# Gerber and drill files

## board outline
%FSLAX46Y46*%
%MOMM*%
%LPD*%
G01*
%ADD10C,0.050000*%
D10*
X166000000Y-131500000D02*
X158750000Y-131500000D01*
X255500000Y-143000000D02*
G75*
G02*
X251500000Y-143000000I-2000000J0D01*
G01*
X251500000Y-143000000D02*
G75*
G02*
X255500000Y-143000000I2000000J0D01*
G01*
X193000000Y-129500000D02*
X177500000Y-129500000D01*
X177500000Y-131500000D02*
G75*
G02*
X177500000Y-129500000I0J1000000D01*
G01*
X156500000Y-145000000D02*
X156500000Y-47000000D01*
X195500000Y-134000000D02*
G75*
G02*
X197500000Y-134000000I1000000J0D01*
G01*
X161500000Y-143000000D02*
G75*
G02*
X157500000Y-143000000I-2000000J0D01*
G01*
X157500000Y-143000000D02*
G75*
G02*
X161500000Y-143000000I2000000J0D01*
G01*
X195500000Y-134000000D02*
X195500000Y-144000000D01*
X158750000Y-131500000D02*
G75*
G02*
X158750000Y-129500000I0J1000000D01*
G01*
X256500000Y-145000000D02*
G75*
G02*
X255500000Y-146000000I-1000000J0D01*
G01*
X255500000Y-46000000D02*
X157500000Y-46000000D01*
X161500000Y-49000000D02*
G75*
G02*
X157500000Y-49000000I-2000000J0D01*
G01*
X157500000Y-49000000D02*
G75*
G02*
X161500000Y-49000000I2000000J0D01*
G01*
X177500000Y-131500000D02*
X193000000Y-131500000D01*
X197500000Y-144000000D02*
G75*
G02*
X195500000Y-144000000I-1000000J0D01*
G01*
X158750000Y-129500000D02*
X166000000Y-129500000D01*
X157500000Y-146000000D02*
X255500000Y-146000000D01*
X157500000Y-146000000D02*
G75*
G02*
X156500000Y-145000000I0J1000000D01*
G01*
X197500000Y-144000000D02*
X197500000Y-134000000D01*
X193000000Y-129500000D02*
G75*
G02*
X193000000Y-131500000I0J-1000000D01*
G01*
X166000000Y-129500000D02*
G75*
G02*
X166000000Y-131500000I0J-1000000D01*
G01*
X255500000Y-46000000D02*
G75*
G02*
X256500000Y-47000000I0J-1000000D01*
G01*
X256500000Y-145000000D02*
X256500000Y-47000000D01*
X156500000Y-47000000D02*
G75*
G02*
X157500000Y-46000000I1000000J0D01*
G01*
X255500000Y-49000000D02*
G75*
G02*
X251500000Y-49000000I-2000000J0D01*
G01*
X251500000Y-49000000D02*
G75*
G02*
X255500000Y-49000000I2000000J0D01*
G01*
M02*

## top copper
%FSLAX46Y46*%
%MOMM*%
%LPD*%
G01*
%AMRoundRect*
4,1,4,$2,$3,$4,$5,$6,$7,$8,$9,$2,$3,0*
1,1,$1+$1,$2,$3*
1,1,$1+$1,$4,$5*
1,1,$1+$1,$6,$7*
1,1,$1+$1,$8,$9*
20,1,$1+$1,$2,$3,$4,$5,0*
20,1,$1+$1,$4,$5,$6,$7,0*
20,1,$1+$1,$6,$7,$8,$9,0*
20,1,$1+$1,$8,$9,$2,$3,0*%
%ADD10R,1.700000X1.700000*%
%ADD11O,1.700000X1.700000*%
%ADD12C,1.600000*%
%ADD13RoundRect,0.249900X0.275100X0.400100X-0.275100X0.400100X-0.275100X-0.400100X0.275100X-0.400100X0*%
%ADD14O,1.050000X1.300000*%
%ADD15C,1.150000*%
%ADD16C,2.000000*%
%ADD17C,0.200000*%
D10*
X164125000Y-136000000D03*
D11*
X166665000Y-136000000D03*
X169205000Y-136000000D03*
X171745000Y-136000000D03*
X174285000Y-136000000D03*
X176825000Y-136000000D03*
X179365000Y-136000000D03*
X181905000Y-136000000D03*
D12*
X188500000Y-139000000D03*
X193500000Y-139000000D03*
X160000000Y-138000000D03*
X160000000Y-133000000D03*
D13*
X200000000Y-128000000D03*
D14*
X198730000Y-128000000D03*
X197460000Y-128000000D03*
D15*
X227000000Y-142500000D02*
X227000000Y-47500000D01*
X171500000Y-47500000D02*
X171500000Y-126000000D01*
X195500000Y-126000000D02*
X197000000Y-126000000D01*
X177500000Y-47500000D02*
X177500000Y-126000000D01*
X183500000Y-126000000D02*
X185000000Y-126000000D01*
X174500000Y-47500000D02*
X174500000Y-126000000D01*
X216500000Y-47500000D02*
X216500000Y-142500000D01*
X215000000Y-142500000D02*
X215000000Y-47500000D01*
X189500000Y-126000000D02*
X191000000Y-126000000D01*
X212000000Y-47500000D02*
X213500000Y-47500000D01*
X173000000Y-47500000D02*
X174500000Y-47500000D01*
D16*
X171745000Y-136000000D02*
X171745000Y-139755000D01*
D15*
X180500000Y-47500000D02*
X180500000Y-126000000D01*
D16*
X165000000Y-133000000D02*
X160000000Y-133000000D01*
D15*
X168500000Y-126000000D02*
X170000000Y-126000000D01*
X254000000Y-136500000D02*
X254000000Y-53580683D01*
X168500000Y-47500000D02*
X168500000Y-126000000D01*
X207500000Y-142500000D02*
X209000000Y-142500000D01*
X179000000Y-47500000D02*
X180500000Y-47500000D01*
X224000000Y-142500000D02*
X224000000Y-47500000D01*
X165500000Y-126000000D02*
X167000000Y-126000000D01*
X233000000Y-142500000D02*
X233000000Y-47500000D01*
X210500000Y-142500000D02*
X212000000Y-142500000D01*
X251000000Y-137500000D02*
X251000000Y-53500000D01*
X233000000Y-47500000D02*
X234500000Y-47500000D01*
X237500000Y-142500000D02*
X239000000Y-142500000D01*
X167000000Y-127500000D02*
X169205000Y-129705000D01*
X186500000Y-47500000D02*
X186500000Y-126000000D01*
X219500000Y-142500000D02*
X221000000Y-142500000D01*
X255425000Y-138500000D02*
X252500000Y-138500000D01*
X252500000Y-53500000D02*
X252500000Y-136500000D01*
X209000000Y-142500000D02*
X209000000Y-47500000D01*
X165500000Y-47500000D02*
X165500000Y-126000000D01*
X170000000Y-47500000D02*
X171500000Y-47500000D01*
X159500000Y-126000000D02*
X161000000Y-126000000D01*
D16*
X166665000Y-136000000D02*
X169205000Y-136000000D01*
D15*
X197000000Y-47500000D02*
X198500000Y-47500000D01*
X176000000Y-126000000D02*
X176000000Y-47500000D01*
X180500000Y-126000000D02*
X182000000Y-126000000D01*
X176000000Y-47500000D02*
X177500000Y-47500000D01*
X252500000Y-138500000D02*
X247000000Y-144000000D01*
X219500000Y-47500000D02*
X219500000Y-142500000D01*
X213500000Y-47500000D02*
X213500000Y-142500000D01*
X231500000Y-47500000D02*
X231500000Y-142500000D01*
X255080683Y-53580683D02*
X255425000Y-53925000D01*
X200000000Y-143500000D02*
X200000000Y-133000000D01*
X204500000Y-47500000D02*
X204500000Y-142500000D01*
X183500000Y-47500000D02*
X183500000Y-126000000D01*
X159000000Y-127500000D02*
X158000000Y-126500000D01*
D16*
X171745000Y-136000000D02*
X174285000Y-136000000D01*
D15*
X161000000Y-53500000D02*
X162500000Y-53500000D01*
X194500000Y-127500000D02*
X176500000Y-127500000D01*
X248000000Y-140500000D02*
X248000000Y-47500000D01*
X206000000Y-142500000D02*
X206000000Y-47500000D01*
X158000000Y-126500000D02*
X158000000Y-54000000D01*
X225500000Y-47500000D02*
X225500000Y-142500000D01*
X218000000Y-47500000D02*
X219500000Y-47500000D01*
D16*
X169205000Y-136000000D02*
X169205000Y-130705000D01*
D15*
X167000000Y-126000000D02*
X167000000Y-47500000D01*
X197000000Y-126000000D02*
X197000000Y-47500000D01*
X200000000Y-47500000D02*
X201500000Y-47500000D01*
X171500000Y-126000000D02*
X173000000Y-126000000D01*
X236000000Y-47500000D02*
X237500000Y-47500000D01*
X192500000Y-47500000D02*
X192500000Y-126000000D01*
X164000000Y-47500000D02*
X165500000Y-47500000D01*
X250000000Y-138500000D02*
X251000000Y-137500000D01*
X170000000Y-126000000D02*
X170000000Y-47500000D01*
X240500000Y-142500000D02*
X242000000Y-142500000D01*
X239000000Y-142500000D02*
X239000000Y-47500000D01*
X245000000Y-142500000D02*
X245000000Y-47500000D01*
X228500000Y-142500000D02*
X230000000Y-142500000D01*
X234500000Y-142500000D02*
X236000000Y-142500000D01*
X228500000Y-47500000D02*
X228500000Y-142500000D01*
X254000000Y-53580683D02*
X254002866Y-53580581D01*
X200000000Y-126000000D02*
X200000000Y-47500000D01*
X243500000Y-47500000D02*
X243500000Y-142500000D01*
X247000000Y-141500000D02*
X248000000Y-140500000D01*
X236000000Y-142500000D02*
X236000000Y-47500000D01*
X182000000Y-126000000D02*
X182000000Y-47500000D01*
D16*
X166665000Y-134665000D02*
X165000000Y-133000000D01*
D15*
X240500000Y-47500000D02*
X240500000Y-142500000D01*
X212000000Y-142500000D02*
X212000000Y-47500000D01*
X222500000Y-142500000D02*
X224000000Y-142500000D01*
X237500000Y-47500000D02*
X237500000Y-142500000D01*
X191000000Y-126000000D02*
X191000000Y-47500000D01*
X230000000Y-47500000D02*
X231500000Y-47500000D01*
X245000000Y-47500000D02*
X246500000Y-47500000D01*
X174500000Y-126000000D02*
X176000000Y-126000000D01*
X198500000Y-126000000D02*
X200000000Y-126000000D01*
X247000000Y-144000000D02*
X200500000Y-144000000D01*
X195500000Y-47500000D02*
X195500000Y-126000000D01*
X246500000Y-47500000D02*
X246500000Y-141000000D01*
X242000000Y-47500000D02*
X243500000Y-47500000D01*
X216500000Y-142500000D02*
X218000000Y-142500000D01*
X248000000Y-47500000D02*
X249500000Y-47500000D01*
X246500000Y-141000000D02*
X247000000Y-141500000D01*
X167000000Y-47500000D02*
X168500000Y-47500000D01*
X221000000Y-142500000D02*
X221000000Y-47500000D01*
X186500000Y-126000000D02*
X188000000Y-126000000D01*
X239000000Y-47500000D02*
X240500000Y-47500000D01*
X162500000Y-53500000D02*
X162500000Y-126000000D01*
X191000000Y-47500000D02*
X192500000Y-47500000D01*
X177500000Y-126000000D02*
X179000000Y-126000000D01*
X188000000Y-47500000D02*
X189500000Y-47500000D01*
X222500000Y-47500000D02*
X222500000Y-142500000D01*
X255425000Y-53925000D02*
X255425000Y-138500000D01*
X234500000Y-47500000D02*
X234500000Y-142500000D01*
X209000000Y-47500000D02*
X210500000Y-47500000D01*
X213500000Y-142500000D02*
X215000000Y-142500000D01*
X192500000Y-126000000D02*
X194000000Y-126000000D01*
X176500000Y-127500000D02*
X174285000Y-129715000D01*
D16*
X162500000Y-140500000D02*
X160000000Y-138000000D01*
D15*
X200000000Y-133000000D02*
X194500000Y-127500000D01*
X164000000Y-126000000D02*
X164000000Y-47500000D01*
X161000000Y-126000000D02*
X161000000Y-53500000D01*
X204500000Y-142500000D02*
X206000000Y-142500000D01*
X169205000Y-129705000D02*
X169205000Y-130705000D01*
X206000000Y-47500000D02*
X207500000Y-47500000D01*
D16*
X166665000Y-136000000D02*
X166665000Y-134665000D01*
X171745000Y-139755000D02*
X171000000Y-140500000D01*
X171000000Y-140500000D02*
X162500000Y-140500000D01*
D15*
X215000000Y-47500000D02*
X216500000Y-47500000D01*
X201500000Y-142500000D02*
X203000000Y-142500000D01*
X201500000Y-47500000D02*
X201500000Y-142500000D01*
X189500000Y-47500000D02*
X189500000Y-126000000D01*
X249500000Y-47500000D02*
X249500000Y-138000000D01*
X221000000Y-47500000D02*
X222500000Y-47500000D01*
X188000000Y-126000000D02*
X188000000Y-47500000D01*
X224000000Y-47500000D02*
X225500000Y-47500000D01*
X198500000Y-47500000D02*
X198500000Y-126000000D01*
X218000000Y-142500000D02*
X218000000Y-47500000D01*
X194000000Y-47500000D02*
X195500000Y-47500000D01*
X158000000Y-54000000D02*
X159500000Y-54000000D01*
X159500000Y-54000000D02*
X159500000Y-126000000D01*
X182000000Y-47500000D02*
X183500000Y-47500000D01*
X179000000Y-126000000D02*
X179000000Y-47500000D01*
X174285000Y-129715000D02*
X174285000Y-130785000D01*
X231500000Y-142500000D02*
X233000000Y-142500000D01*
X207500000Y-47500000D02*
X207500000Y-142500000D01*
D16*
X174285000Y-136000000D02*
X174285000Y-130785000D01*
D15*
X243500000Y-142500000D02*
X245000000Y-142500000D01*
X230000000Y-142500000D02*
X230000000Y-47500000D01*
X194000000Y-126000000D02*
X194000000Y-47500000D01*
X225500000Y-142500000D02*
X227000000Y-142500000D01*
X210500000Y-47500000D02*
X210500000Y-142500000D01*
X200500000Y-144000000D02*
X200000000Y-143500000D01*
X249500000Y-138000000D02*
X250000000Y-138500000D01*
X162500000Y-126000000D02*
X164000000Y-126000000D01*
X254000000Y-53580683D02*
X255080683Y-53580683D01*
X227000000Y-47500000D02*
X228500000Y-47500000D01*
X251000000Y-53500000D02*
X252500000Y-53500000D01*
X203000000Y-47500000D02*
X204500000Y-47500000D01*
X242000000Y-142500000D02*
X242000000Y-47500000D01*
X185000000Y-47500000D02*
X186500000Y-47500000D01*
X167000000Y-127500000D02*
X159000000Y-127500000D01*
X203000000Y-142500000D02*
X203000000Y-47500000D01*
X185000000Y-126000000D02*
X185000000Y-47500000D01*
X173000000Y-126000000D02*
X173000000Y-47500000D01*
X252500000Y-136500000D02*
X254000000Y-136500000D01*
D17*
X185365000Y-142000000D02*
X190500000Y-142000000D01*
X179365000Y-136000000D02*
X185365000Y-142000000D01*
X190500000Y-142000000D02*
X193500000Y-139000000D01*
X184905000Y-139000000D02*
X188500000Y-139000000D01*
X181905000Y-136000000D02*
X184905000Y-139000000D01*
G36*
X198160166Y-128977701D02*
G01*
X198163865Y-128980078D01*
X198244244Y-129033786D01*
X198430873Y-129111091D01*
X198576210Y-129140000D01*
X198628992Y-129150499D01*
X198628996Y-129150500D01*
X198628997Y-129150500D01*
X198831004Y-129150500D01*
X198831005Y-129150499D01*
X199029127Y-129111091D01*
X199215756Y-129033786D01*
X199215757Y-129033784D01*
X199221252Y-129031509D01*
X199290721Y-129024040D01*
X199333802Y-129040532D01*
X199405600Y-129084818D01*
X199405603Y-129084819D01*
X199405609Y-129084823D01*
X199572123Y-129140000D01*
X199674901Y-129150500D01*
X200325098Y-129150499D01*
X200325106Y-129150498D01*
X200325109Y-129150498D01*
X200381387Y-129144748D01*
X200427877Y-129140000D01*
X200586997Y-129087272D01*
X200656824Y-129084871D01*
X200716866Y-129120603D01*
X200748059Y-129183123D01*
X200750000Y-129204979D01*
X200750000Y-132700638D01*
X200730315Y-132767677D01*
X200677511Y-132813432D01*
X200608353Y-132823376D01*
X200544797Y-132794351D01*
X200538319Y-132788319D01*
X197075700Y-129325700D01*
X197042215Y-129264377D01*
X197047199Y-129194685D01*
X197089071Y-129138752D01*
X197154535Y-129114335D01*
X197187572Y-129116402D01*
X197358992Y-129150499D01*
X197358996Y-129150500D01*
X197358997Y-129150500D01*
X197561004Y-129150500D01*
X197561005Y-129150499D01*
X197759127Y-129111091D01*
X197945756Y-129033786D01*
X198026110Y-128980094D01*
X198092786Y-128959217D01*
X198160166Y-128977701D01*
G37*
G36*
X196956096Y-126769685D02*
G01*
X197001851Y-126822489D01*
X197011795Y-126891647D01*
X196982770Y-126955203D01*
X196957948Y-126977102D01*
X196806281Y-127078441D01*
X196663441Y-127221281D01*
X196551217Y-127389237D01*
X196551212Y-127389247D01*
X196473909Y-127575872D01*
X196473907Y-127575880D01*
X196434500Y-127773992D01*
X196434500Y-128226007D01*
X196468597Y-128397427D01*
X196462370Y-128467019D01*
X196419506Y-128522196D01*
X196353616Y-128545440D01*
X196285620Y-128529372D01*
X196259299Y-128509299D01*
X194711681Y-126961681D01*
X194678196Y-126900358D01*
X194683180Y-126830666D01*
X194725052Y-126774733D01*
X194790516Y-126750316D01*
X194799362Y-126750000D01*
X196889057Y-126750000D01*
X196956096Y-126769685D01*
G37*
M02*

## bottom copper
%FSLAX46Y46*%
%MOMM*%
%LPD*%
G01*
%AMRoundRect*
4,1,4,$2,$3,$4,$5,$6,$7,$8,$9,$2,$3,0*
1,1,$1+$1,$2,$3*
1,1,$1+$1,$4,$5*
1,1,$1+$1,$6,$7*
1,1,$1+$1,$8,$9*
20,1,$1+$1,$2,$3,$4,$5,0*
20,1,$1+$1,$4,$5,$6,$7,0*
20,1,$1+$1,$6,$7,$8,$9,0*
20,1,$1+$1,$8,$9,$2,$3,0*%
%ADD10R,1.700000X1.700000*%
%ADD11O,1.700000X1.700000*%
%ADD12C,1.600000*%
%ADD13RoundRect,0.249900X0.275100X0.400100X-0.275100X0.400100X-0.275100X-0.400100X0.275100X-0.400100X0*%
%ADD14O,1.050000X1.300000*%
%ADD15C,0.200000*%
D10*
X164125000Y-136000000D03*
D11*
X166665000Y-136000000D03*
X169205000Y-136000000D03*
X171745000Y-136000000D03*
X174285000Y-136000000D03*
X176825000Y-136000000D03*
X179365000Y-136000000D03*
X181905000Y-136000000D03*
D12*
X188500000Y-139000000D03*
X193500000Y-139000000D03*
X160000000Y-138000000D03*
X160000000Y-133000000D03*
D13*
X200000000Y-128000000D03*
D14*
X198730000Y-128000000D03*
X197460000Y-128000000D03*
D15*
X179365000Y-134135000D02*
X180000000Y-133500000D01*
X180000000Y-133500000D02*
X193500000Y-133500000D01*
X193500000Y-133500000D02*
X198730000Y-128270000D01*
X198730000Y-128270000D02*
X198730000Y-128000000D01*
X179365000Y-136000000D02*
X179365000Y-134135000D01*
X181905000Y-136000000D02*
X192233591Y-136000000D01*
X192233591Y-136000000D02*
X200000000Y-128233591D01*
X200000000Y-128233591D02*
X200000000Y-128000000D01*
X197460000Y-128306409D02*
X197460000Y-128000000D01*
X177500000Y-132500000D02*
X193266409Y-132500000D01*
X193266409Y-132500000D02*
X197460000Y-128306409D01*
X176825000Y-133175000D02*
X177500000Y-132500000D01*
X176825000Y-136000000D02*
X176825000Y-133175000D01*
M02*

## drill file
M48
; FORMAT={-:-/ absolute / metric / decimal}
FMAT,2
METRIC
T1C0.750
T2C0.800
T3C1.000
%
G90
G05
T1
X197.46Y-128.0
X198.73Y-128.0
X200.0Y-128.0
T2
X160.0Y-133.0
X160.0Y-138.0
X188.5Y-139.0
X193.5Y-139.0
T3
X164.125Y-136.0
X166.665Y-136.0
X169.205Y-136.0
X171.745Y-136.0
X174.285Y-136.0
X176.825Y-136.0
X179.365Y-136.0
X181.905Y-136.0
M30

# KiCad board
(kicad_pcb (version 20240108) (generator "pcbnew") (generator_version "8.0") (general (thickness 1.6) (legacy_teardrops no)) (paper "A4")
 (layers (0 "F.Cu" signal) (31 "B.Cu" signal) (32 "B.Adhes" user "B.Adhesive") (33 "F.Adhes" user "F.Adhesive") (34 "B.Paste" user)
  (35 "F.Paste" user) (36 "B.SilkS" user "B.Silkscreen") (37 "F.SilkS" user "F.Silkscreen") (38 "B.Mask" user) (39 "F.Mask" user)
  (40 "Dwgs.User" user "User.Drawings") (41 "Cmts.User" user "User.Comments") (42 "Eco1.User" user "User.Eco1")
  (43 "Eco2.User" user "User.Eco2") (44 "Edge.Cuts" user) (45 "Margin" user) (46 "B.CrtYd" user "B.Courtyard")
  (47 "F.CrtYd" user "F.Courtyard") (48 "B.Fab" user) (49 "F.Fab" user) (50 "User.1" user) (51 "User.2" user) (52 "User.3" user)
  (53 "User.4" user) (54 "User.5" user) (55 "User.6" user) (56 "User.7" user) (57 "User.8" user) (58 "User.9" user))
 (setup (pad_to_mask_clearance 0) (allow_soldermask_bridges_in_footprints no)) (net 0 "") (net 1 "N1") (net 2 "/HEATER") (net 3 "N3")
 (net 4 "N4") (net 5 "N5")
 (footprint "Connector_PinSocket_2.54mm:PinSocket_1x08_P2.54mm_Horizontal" (layer "F.Cu") (at 164.125 136 90)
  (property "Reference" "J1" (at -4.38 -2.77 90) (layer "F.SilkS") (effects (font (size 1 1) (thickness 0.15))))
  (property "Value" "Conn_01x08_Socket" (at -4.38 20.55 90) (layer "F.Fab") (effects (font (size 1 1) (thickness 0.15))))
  (pad "1" thru_hole rect (at 0 0 90) (size 1.7 1.7) (drill 1) (layers "*.Cu" "*.Mask") (remove_unused_layers no) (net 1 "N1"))
  (pad "2" thru_hole oval (at 0 2.54 90) (size 1.7 1.7) (drill 1) (layers "*.Cu" "*.Mask") (remove_unused_layers no) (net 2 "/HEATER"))
  (pad "3" thru_hole oval (at 0 5.08 90) (size 1.7 1.7) (drill 1) (layers "*.Cu" "*.Mask") (remove_unused_layers no) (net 2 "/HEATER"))
  (pad "4" thru_hole oval (at 0 7.62 90) (size 1.7 1.7) (drill 1) (layers "*.Cu" "*.Mask") (remove_unused_layers no) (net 2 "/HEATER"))
  (pad "5" thru_hole oval (at 0 10.16 90) (size 1.7 1.7) (drill 1) (layers "*.Cu" "*.Mask") (remove_unused_layers no) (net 2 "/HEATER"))
  (pad "6" thru_hole oval (at 0 12.7 90) (size 1.7 1.7) (drill 1) (layers "*.Cu" "*.Mask") (remove_unused_layers no) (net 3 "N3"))
  (pad "7" thru_hole oval (at 0 15.24 90) (size 1.7 1.7) (drill 1) (layers "*.Cu" "*.Mask") (remove_unused_layers no) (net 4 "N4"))
  (pad "8" thru_hole oval (at 0 17.78 90) (size 1.7 1.7) (drill 1) (layers "*.Cu" "*.Mask") (remove_unused_layers no) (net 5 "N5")))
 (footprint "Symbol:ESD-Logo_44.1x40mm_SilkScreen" (layer "F.Cu") (at 207.5 88.5)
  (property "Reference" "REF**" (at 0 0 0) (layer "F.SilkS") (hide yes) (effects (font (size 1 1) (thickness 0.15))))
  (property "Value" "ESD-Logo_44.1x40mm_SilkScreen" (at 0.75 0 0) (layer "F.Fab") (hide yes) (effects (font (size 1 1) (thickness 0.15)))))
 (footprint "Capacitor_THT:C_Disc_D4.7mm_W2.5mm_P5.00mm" (layer "F.Cu") (at 188.5 139)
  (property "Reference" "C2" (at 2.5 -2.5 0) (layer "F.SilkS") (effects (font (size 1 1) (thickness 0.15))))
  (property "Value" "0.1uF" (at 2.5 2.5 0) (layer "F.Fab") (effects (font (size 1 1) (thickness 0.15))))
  (pad "1" thru_hole circle (at 0 0) (size 1.6 1.6) (drill 0.8) (layers "*.Cu" "*.Mask") (remove_unused_layers no) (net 4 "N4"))
  (pad "2" thru_hole circle (at 5 0) (size 1.6 1.6) (drill 0.8) (layers "*.Cu" "*.Mask") (remove_unused_layers no) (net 3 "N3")))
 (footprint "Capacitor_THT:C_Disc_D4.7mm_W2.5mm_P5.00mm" (layer "F.Cu") (at 160 138 90)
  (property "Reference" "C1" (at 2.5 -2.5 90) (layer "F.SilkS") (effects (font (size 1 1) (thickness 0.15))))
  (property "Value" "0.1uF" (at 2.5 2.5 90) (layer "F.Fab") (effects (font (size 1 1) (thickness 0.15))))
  (pad "1" thru_hole circle (at 0 0 90) (size 1.6 1.6) (drill 0.8) (layers "*.Cu" "*.Mask") (remove_unused_layers no) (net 2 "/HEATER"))
  (pad "2" thru_hole circle (at 5 0 90) (size 1.6 1.6) (drill 0.8) (layers "*.Cu" "*.Mask") (remove_unused_layers no) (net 2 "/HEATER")))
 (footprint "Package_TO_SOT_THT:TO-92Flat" (layer "F.Cu") (at 200 128 180)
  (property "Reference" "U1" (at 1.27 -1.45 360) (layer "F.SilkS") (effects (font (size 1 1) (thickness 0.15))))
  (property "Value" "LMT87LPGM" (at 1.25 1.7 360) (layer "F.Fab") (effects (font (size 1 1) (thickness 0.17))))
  (pad "1" thru_hole roundrect (at 0 0 180) (size 1.05 1.3) (drill 0.75) (layers "*.Cu" "*.Mask") (remove_unused_layers no)
   (roundrect_rratio 0.238) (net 5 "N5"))
  (pad "2" thru_hole oval (at 1.27 0 180) (size 1.05 1.3) (drill 0.75) (layers "*.Cu" "*.Mask") (remove_unused_layers no) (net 4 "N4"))
  (pad "3" thru_hole oval (at 2.54 0 180) (size 1.05 1.3) (drill 0.75) (layers "*.Cu" "*.Mask") (remove_unused_layers no) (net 3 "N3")))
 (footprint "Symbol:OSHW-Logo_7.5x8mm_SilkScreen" (layer "B.Cu") (at 222.5 140 180)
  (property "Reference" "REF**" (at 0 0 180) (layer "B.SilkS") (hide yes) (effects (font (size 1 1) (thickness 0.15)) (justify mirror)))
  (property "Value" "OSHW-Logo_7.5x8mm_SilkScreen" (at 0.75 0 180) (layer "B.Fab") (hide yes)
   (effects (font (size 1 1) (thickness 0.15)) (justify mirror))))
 (gr_line (start 166 131.5) (end 158.75 131.5) (stroke (width 0.05) (type default)) (layer "Edge.Cuts"))
 (gr_circle (center 253.5 143) (end 253.5 141) (stroke (width 0.05) (type default)) (fill none) (layer "Edge.Cuts"))
 (gr_line (start 193 129.5) (end 177.5 129.5) (stroke (width 0.05) (type default)) (layer "Edge.Cuts"))
 (gr_arc (start 177.5 131.5) (mid 176.5 130.5) (end 177.5 129.5) (stroke (width 0.05) (type default)) (layer "Edge.Cuts"))
 (gr_line (start 156.5 145) (end 156.5 47) (stroke (width 0.05) (type default)) (layer "Edge.Cuts"))
 (gr_arc (start 195.5 134) (mid 196.5 133) (end 197.5 134) (stroke (width 0.05) (type default)) (layer "Edge.Cuts"))
 (gr_circle (center 159.5 143) (end 159.5 141) (stroke (width 0.05) (type default)) (fill none) (layer "Edge.Cuts"))
 (gr_line (start 195.5 134) (end 195.5 144) (stroke (width 0.05) (type default)) (layer "Edge.Cuts"))
 (gr_arc (start 158.75 131.5) (mid 157.75 130.5) (end 158.75 129.5) (stroke (width 0.05) (type default)) (layer "Edge.Cuts"))
 (gr_arc (start 256.5 145) (mid 256.207107 145.707107) (end 255.5 146) (stroke (width 0.05) (type default)) (layer "Edge.Cuts"))
 (gr_line (start 255.5 46) (end 157.5 46) (stroke (width 0.05) (type default)) (layer "Edge.Cuts"))
 (gr_circle (center 159.5 49) (end 159.5 47) (stroke (width 0.05) (type default)) (fill none) (layer "Edge.Cuts"))
 (gr_line (start 177.5 131.5) (end 193 131.5) (stroke (width 0.05) (type default)) (layer "Edge.Cuts"))
 (gr_arc (start 197.5 144) (mid 196.5 145) (end 195.5 144) (stroke (width 0.05) (type default)) (layer "Edge.Cuts"))
 (gr_line (start 158.75 129.5) (end 166 129.5) (stroke (width 0.05) (type default)) (layer "Edge.Cuts"))
 (gr_line (start 157.5 146) (end 255.5 146) (stroke (width 0.05) (type default)) (layer "Edge.Cuts"))
 (gr_arc (start 157.5 146) (mid 156.792893 145.707107) (end 156.5 145) (stroke (width 0.05) (type default)) (layer "Edge.Cuts"))
 (gr_line (start 197.5 144) (end 197.5 134) (stroke (width 0.05) (type default)) (layer "Edge.Cuts"))
 (gr_arc (start 193 129.5) (mid 194 130.5) (end 193 131.5) (stroke (width 0.05) (type default)) (layer "Edge.Cuts"))
 (gr_arc (start 166 129.5) (mid 167 130.5) (end 166 131.5) (stroke (width 0.05) (type default)) (layer "Edge.Cuts"))
 (gr_arc (start 255.5 46) (mid 256.207107 46.292893) (end 256.5 47) (stroke (width 0.05) (type default)) (layer "Edge.Cuts"))
 (gr_line (start 256.5 145) (end 256.5 47) (stroke (width 0.05) (type default)) (layer "Edge.Cuts"))
 (gr_arc (start 156.5 47) (mid 156.792893 46.292893) (end 157.5 46) (stroke (width 0.05) (type default)) (layer "Edge.Cuts"))
 (gr_circle (center 253.5 49) (end 253.5 47) (stroke (width 0.05) (type default)) (fill none) (layer "Edge.Cuts"))
 (segment (start 227 142.5) (end 227 47.5) (width 1.15) (layer "F.Cu") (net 2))
 (segment (start 171.5 47.5) (end 171.5 126) (width 1.15) (layer "F.Cu") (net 2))
 (segment (start 195.5 126) (end 197 126) (width 1.15) (layer "F.Cu") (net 2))
 (segment (start 177.5 47.5) (end 177.5 126) (width 1.15) (layer "F.Cu") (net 2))
 (segment (start 183.5 126) (end 185 126) (width 1.15) (layer "F.Cu") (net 2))
 (segment (start 174.5 47.5) (end 174.5 126) (width 1.15) (layer "F.Cu") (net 2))
 (segment (start 216.5 47.5) (end 216.5 142.5) (width 1.15) (layer "F.Cu") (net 2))
 (segment (start 215 142.5) (end 215 47.5) (width 1.15) (layer "F.Cu") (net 2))
 (segment (start 189.5 126) (end 191 126) (width 1.15) (layer "F.Cu") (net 2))
 (segment (start 212 47.5) (end 213.5 47.5) (width 1.15) (layer "F.Cu") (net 2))
 (segment (start 173 47.5) (end 174.5 47.5) (width 1.15) (layer "F.Cu") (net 2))
 (segment (start 171.745 136) (end 171.745 139.755) (width 2) (layer "F.Cu") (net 2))
 (segment (start 180.5 47.5) (end 180.5 126) (width 1.15) (layer "F.Cu") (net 2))
 (segment (start 165 133) (end 160 133) (width 2) (layer "F.Cu") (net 2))
 (segment (start 168.5 126) (end 170 126) (width 1.15) (layer "F.Cu") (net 2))
 (segment (start 254 136.5) (end 254 53.580683) (width 1.15) (layer "F.Cu") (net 2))
 (segment (start 168.5 47.5) (end 168.5 126) (width 1.15) (layer "F.Cu") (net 2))
 (segment (start 207.5 142.5) (end 209 142.5) (width 1.15) (layer "F.Cu") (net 2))
 (segment (start 179 47.5) (end 180.5 47.5) (width 1.15) (layer "F.Cu") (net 2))
 (segment (start 224 142.5) (end 224 47.5) (width 1.15) (layer "F.Cu") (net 2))
 (segment (start 165.5 126) (end 167 126) (width 1.15) (layer "F.Cu") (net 2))
 (segment (start 233 142.5) (end 233 47.5) (width 1.15) (layer "F.Cu") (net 2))
 (segment (start 210.5 142.5) (end 212 142.5) (width 1.15) (layer "F.Cu") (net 2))
 (segment (start 251 137.5) (end 251 53.5) (width 1.15) (layer "F.Cu") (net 2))
 (segment (start 233 47.5) (end 234.5 47.5) (width 1.15) (layer "F.Cu") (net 2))
 (segment (start 237.5 142.5) (end 239 142.5) (width 1.15) (layer "F.Cu") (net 2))
 (segment (start 167 127.5) (end 169.205 129.705) (width 1.15) (layer "F.Cu") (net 2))
 (segment (start 186.5 47.5) (end 186.5 126) (width 1.15) (layer "F.Cu") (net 2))
 (segment (start 219.5 142.5) (end 221 142.5) (width 1.15) (layer "F.Cu") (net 2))
 (segment (start 255.425 138.5) (end 252.5 138.5) (width 1.15) (layer "F.Cu") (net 2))
 (segment (start 252.5 53.5) (end 252.5 136.5) (width 1.15) (layer "F.Cu") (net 2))
 (segment (start 209 142.5) (end 209 47.5) (width 1.15) (layer "F.Cu") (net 2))
 (segment (start 165.5 47.5) (end 165.5 126) (width 1.15) (layer "F.Cu") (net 2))
 (segment (start 170 47.5) (end 171.5 47.5) (width 1.15) (layer "F.Cu") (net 2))
 (segment (start 159.5 126) (end 161 126) (width 1.15) (layer "F.Cu") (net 2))
 (segment (start 166.665 136) (end 169.205 136) (width 2) (layer "F.Cu") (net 2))
 (segment (start 197 47.5) (end 198.5 47.5) (width 1.15) (layer "F.Cu") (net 2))
 (segment (start 176 126) (end 176 47.5) (width 1.15) (layer "F.Cu") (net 2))
 (segment (start 180.5 126) (end 182 126) (width 1.15) (layer "F.Cu") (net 2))
 (segment (start 176 47.5) (end 177.5 47.5) (width 1.15) (layer "F.Cu") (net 2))
 (segment (start 252.5 138.5) (end 247 144) (width 1.15) (layer "F.Cu") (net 2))
 (segment (start 219.5 47.5) (end 219.5 142.5) (width 1.15) (layer "F.Cu") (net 2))
 (segment (start 213.5 47.5) (end 213.5 142.5) (width 1.15) (layer "F.Cu") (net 2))
 (segment (start 231.5 47.5) (end 231.5 142.5) (width 1.15) (layer "F.Cu") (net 2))
 (segment (start 255.080683 53.580683) (end 255.425 53.925) (width 1.15) (layer "F.Cu") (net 2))
 (segment (start 200 143.5) (end 200 133) (width 1.15) (layer "F.Cu") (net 2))
 (segment (start 204.5 47.5) (end 204.5 142.5) (width 1.15) (layer "F.Cu") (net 2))
 (segment (start 183.5 47.5) (end 183.5 126) (width 1.15) (layer "F.Cu") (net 2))
 (segment (start 159 127.5) (end 158 126.5) (width 1.15) (layer "F.Cu") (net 2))
 (segment (start 171.745 136) (end 174.285 136) (width 2) (layer "F.Cu") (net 2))
 (segment (start 161 53.5) (end 162.5 53.5) (width 1.15) (layer "F.Cu") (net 2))
 (segment (start 194.5 127.5) (end 176.5 127.5) (width 1.15) (layer "F.Cu") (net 2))
 (segment (start 248 140.5) (end 248 47.5) (width 1.15) (layer "F.Cu") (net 2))
 (segment (start 206 142.5) (end 206 47.5) (width 1.15) (layer "F.Cu") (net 2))
 (segment (start 158 126.5) (end 158 54) (width 1.15) (layer "F.Cu") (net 2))
 (segment (start 225.5 47.5) (end 225.5 142.5) (width 1.15) (layer "F.Cu") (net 2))
 (segment (start 218 47.5) (end 219.5 47.5) (width 1.15) (layer "F.Cu") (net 2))
 (segment (start 169.205 136) (end 169.205 130.705) (width 2) (layer "F.Cu") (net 2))
 (segment (start 167 126) (end 167 47.5) (width 1.15) (layer "F.Cu") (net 2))
 (segment (start 197 126) (end 197 47.5) (width 1.15) (layer "F.Cu") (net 2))
 (segment (start 200 47.5) (end 201.5 47.5) (width 1.15) (layer "F.Cu") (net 2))
 (segment (start 171.5 126) (end 173 126) (width 1.15) (layer "F.Cu") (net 2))
 (segment (start 236 47.5) (end 237.5 47.5) (width 1.15) (layer "F.Cu") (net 2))
 (segment (start 192.5 47.5) (end 192.5 126) (width 1.15) (layer "F.Cu") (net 2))
 (segment (start 164 47.5) (end 165.5 47.5) (width 1.15) (layer "F.Cu") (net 2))
 (segment (start 250 138.5) (end 251 137.5) (width 1.15) (layer "F.Cu") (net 2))
 (segment (start 170 126) (end 170 47.5) (width 1.15) (layer "F.Cu") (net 2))
 (segment (start 240.5 142.5) (end 242 142.5) (width 1.15) (layer "F.Cu") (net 2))
 (segment (start 239 142.5) (end 239 47.5) (width 1.15) (layer "F.Cu") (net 2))
 (segment (start 245 142.5) (end 245 47.5) (width 1.15) (layer "F.Cu") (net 2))
 (segment (start 228.5 142.5) (end 230 142.5) (width 1.15) (layer "F.Cu") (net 2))
 (segment (start 234.5 142.5) (end 236 142.5) (width 1.15) (layer "F.Cu") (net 2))
 (segment (start 228.5 47.5) (end 228.5 142.5) (width 1.15) (layer "F.Cu") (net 2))
 (segment (start 254 53.580683) (end 254.002866 53.580581) (width 1.15) (layer "F.Cu") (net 2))
 (segment (start 200 126) (end 200 47.5) (width 1.15) (layer "F.Cu") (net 2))
 (segment (start 243.5 47.5) (end 243.5 142.5) (width 1.15) (layer "F.Cu") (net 2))
 (segment (start 247 141.5) (end 248 140.5) (width 1.15) (layer "F.Cu") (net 2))
 (segment (start 236 142.5) (end 236 47.5) (width 1.15) (layer "F.Cu") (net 2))
 (segment (start 182 126) (end 182 47.5) (width 1.15) (layer "F.Cu") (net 2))
 (segment (start 166.665 134.665) (end 165 133) (width 2) (layer "F.Cu") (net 2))
 (segment (start 240.5 47.5) (end 240.5 142.5) (width 1.15) (layer "F.Cu") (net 2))
 (segment (start 212 142.5) (end 212 47.5) (width 1.15) (layer "F.Cu") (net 2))
 (segment (start 222.5 142.5) (end 224 142.5) (width 1.15) (layer "F.Cu") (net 2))
 (segment (start 237.5 47.5) (end 237.5 142.5) (width 1.15) (layer "F.Cu") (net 2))
 (segment (start 191 126) (end 191 47.5) (width 1.15) (layer "F.Cu") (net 2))
 (segment (start 230 47.5) (end 231.5 47.5) (width 1.15) (layer "F.Cu") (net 2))
 (segment (start 245 47.5) (end 246.5 47.5) (width 1.15) (layer "F.Cu") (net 2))
 (segment (start 174.5 126) (end 176 126) (width 1.15) (layer "F.Cu") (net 2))
 (segment (start 198.5 126) (end 200 126) (width 1.15) (layer "F.Cu") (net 2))
 (segment (start 247 144) (end 200.5 144) (width 1.15) (layer "F.Cu") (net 2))
 (segment (start 195.5 47.5) (end 195.5 126) (width 1.15) (layer "F.Cu") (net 2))
 (segment (start 246.5 47.5) (end 246.5 141) (width 1.15) (layer "F.Cu") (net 2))
 (segment (start 242 47.5) (end 243.5 47.5) (width 1.15) (layer "F.Cu") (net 2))
 (segment (start 216.5 142.5) (end 218 142.5) (width 1.15) (layer "F.Cu") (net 2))
 (segment (start 248 47.5) (end 249.5 47.5) (width 1.15) (layer "F.Cu") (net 2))
 (segment (start 246.5 141) (end 247 141.5) (width 1.15) (layer "F.Cu") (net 2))
 (segment (start 167 47.5) (end 168.5 47.5) (width 1.15) (layer "F.Cu") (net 2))
 (segment (start 221 142.5) (end 221 47.5) (width 1.15) (layer "F.Cu") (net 2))
 (segment (start 186.5 126) (end 188 126) (width 1.15) (layer "F.Cu") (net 2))
 (segment (start 239 47.5) (end 240.5 47.5) (width 1.15) (layer "F.Cu") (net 2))
 (segment (start 162.5 53.5) (end 162.5 126) (width 1.15) (layer "F.Cu") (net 2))
 (segment (start 191 47.5) (end 192.5 47.5) (width 1.15) (layer "F.Cu") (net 2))
 (segment (start 177.5 126) (end 179 126) (width 1.15) (layer "F.Cu") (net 2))
 (segment (start 188 47.5) (end 189.5 47.5) (width 1.15) (layer "F.Cu") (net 2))
 (segment (start 222.5 47.5) (end 222.5 142.5) (width 1.15) (layer "F.Cu") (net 2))
 (segment (start 255.425 53.925) (end 255.425 138.5) (width 1.15) (layer "F.Cu") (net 2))
 (segment (start 234.5 47.5) (end 234.5 142.5) (width 1.15) (layer "F.Cu") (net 2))
 (segment (start 209 47.5) (end 210.5 47.5) (width 1.15) (layer "F.Cu") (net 2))
 (segment (start 213.5 142.5) (end 215 142.5) (width 1.15) (layer "F.Cu") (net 2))
 (segment (start 192.5 126) (end 194 126) (width 1.15) (layer "F.Cu") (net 2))
 (segment (start 176.5 127.5) (end 174.285 129.715) (width 1.15) (layer "F.Cu") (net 2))
 (segment (start 162.5 140.5) (end 160 138) (width 2) (layer "F.Cu") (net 2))
 (segment (start 200 133) (end 194.5 127.5) (width 1.15) (layer "F.Cu") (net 2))
 (segment (start 164 126) (end 164 47.5) (width 1.15) (layer "F.Cu") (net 2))
 (segment (start 161 126) (end 161 53.5) (width 1.15) (layer "F.Cu") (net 2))
 (segment (start 204.5 142.5) (end 206 142.5) (width 1.15) (layer "F.Cu") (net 2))
 (segment (start 169.205 129.705) (end 169.205 130.705) (width 1.15) (layer "F.Cu") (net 2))
 (segment (start 206 47.5) (end 207.5 47.5) (width 1.15) (layer "F.Cu") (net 2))
 (segment (start 166.665 136) (end 166.665 134.665) (width 2) (layer "F.Cu") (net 2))
 (segment (start 171.745 139.755) (end 171 140.5) (width 2) (layer "F.Cu") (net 2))
 (segment (start 171 140.5) (end 162.5 140.5) (width 2) (layer "F.Cu") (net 2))
 (segment (start 215 47.5) (end 216.5 47.5) (width 1.15) (layer "F.Cu") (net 2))
 (segment (start 201.5 142.5) (end 203 142.5) (width 1.15) (layer "F.Cu") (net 2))
 (segment (start 201.5 47.5) (end 201.5 142.5) (width 1.15) (layer "F.Cu") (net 2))
 (segment (start 189.5 47.5) (end 189.5 126) (width 1.15) (layer "F.Cu") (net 2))
 (segment (start 249.5 47.5) (end 249.5 138) (width 1.15) (layer "F.Cu") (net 2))
 (segment (start 221 47.5) (end 222.5 47.5) (width 1.15) (layer "F.Cu") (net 2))
 (segment (start 188 126) (end 188 47.5) (width 1.15) (layer "F.Cu") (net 2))
 (segment (start 224 47.5) (end 225.5 47.5) (width 1.15) (layer "F.Cu") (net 2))
 (segment (start 198.5 47.5) (end 198.5 126) (width 1.15) (layer "F.Cu") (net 2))
 (segment (start 218 142.5) (end 218 47.5) (width 1.15) (layer "F.Cu") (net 2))
 (segment (start 194 47.5) (end 195.5 47.5) (width 1.15) (layer "F.Cu") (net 2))
 (segment (start 158 54) (end 159.5 54) (width 1.15) (layer "F.Cu") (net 2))
 (segment (start 159.5 54) (end 159.5 126) (width 1.15) (layer "F.Cu") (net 2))
 (segment (start 182 47.5) (end 183.5 47.5) (width 1.15) (layer "F.Cu") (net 2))
 (segment (start 179 126) (end 179 47.5) (width 1.15) (layer "F.Cu") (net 2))
 (segment (start 174.285 129.715) (end 174.285 130.785) (width 1.15) (layer "F.Cu") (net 2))
 (segment (start 231.5 142.5) (end 233 142.5) (width 1.15) (layer "F.Cu") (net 2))
 (segment (start 207.5 47.5) (end 207.5 142.5) (width 1.15) (layer "F.Cu") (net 2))
 (segment (start 174.285 136) (end 174.285 130.785) (width 2) (layer "F.Cu") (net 2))
 (segment (start 243.5 142.5) (end 245 142.5) (width 1.15) (layer "F.Cu") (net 2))
 (segment (start 230 142.5) (end 230 47.5) (width 1.15) (layer "F.Cu") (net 2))
 (segment (start 194 126) (end 194 47.5) (width 1.15) (layer "F.Cu") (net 2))
 (segment (start 225.5 142.5) (end 227 142.5) (width 1.15) (layer "F.Cu") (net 2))
 (segment (start 210.5 47.5) (end 210.5 142.5) (width 1.15) (layer "F.Cu") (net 2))
 (segment (start 200.5 144) (end 200 143.5) (width 1.15) (layer "F.Cu") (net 2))
 (segment (start 249.5 138) (end 250 138.5) (width 1.15) (layer "F.Cu") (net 2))
 (segment (start 162.5 126) (end 164 126) (width 1.15) (layer "F.Cu") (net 2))
 (segment (start 254 53.580683) (end 255.080683 53.580683) (width 1.15) (layer "F.Cu") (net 2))
 (segment (start 227 47.5) (end 228.5 47.5) (width 1.15) (layer "F.Cu") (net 2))
 (segment (start 251 53.5) (end 252.5 53.5) (width 1.15) (layer "F.Cu") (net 2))
 (segment (start 203 47.5) (end 204.5 47.5) (width 1.15) (layer "F.Cu") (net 2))
 (segment (start 242 142.5) (end 242 47.5) (width 1.15) (layer "F.Cu") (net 2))
 (segment (start 185 47.5) (end 186.5 47.5) (width 1.15) (layer "F.Cu") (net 2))
 (segment (start 167 127.5) (end 159 127.5) (width 1.15) (layer "F.Cu") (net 2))
 (segment (start 203 142.5) (end 203 47.5) (width 1.15) (layer "F.Cu") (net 2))
 (segment (start 185 126) (end 185 47.5) (width 1.15) (layer "F.Cu") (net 2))
 (segment (start 173 126) (end 173 47.5) (width 1.15) (layer "F.Cu") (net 2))
 (segment (start 252.5 136.5) (end 254 136.5) (width 1.15) (layer "F.Cu") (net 2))
 (segment (start 185.365 142) (end 190.5 142) (width 0.2) (layer "F.Cu") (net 4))
 (segment (start 179.365 136) (end 185.365 142) (width 0.2) (layer "F.Cu") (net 4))
 (segment (start 190.5 142) (end 193.5 139) (width 0.2) (layer "F.Cu") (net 4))
 (segment (start 179.365 134.135) (end 180 133.5) (width 0.2) (layer "B.Cu") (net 4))
 (segment (start 180 133.5) (end 193.5 133.5) (width 0.2) (layer "B.Cu") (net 4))
 (segment (start 193.5 133.5) (end 198.73 128.27) (width 0.2) (layer "B.Cu") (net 4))
 (segment (start 198.73 128.27) (end 198.73 128) (width 0.2) (layer "B.Cu") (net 4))
 (segment (start 179.365 136) (end 179.365 134.135) (width 0.2) (layer "B.Cu") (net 4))
 (segment (start 184.905 139) (end 188.5 139) (width 0.2) (layer "F.Cu") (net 5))
 (segment (start 181.905 136) (end 184.905 139) (width 0.2) (layer "F.Cu") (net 5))
 (segment (start 181.905 136) (end 192.233591 136) (width 0.2) (layer "B.Cu") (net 5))
 (segment (start 192.233591 136) (end 200 128.233591) (width 0.2) (layer "B.Cu") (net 5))
 (segment (start 200 128.233591) (end 200 128) (width 0.2) (layer "B.Cu") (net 5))
 (segment (start 197.46 128.306409) (end 197.46 128) (width 0.2) (layer "B.Cu") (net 3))
 (segment (start 177.5 132.5) (end 193.266409 132.5) (width 0.2) (layer "B.Cu") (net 3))
 (segment (start 193.266409 132.5) (end 197.46 128.306409) (width 0.2) (layer "B.Cu") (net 3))
 (segment (start 176.825 133.175) (end 177.5 132.5) (width 0.2) (layer "B.Cu") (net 3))
 (segment (start 176.825 136) (end 176.825 133.175) (width 0.2) (layer "B.Cu") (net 3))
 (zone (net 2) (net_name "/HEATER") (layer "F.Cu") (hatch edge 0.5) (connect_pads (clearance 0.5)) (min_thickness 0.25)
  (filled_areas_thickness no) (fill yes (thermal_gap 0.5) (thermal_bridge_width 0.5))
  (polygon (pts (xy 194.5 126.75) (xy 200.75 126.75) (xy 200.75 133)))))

